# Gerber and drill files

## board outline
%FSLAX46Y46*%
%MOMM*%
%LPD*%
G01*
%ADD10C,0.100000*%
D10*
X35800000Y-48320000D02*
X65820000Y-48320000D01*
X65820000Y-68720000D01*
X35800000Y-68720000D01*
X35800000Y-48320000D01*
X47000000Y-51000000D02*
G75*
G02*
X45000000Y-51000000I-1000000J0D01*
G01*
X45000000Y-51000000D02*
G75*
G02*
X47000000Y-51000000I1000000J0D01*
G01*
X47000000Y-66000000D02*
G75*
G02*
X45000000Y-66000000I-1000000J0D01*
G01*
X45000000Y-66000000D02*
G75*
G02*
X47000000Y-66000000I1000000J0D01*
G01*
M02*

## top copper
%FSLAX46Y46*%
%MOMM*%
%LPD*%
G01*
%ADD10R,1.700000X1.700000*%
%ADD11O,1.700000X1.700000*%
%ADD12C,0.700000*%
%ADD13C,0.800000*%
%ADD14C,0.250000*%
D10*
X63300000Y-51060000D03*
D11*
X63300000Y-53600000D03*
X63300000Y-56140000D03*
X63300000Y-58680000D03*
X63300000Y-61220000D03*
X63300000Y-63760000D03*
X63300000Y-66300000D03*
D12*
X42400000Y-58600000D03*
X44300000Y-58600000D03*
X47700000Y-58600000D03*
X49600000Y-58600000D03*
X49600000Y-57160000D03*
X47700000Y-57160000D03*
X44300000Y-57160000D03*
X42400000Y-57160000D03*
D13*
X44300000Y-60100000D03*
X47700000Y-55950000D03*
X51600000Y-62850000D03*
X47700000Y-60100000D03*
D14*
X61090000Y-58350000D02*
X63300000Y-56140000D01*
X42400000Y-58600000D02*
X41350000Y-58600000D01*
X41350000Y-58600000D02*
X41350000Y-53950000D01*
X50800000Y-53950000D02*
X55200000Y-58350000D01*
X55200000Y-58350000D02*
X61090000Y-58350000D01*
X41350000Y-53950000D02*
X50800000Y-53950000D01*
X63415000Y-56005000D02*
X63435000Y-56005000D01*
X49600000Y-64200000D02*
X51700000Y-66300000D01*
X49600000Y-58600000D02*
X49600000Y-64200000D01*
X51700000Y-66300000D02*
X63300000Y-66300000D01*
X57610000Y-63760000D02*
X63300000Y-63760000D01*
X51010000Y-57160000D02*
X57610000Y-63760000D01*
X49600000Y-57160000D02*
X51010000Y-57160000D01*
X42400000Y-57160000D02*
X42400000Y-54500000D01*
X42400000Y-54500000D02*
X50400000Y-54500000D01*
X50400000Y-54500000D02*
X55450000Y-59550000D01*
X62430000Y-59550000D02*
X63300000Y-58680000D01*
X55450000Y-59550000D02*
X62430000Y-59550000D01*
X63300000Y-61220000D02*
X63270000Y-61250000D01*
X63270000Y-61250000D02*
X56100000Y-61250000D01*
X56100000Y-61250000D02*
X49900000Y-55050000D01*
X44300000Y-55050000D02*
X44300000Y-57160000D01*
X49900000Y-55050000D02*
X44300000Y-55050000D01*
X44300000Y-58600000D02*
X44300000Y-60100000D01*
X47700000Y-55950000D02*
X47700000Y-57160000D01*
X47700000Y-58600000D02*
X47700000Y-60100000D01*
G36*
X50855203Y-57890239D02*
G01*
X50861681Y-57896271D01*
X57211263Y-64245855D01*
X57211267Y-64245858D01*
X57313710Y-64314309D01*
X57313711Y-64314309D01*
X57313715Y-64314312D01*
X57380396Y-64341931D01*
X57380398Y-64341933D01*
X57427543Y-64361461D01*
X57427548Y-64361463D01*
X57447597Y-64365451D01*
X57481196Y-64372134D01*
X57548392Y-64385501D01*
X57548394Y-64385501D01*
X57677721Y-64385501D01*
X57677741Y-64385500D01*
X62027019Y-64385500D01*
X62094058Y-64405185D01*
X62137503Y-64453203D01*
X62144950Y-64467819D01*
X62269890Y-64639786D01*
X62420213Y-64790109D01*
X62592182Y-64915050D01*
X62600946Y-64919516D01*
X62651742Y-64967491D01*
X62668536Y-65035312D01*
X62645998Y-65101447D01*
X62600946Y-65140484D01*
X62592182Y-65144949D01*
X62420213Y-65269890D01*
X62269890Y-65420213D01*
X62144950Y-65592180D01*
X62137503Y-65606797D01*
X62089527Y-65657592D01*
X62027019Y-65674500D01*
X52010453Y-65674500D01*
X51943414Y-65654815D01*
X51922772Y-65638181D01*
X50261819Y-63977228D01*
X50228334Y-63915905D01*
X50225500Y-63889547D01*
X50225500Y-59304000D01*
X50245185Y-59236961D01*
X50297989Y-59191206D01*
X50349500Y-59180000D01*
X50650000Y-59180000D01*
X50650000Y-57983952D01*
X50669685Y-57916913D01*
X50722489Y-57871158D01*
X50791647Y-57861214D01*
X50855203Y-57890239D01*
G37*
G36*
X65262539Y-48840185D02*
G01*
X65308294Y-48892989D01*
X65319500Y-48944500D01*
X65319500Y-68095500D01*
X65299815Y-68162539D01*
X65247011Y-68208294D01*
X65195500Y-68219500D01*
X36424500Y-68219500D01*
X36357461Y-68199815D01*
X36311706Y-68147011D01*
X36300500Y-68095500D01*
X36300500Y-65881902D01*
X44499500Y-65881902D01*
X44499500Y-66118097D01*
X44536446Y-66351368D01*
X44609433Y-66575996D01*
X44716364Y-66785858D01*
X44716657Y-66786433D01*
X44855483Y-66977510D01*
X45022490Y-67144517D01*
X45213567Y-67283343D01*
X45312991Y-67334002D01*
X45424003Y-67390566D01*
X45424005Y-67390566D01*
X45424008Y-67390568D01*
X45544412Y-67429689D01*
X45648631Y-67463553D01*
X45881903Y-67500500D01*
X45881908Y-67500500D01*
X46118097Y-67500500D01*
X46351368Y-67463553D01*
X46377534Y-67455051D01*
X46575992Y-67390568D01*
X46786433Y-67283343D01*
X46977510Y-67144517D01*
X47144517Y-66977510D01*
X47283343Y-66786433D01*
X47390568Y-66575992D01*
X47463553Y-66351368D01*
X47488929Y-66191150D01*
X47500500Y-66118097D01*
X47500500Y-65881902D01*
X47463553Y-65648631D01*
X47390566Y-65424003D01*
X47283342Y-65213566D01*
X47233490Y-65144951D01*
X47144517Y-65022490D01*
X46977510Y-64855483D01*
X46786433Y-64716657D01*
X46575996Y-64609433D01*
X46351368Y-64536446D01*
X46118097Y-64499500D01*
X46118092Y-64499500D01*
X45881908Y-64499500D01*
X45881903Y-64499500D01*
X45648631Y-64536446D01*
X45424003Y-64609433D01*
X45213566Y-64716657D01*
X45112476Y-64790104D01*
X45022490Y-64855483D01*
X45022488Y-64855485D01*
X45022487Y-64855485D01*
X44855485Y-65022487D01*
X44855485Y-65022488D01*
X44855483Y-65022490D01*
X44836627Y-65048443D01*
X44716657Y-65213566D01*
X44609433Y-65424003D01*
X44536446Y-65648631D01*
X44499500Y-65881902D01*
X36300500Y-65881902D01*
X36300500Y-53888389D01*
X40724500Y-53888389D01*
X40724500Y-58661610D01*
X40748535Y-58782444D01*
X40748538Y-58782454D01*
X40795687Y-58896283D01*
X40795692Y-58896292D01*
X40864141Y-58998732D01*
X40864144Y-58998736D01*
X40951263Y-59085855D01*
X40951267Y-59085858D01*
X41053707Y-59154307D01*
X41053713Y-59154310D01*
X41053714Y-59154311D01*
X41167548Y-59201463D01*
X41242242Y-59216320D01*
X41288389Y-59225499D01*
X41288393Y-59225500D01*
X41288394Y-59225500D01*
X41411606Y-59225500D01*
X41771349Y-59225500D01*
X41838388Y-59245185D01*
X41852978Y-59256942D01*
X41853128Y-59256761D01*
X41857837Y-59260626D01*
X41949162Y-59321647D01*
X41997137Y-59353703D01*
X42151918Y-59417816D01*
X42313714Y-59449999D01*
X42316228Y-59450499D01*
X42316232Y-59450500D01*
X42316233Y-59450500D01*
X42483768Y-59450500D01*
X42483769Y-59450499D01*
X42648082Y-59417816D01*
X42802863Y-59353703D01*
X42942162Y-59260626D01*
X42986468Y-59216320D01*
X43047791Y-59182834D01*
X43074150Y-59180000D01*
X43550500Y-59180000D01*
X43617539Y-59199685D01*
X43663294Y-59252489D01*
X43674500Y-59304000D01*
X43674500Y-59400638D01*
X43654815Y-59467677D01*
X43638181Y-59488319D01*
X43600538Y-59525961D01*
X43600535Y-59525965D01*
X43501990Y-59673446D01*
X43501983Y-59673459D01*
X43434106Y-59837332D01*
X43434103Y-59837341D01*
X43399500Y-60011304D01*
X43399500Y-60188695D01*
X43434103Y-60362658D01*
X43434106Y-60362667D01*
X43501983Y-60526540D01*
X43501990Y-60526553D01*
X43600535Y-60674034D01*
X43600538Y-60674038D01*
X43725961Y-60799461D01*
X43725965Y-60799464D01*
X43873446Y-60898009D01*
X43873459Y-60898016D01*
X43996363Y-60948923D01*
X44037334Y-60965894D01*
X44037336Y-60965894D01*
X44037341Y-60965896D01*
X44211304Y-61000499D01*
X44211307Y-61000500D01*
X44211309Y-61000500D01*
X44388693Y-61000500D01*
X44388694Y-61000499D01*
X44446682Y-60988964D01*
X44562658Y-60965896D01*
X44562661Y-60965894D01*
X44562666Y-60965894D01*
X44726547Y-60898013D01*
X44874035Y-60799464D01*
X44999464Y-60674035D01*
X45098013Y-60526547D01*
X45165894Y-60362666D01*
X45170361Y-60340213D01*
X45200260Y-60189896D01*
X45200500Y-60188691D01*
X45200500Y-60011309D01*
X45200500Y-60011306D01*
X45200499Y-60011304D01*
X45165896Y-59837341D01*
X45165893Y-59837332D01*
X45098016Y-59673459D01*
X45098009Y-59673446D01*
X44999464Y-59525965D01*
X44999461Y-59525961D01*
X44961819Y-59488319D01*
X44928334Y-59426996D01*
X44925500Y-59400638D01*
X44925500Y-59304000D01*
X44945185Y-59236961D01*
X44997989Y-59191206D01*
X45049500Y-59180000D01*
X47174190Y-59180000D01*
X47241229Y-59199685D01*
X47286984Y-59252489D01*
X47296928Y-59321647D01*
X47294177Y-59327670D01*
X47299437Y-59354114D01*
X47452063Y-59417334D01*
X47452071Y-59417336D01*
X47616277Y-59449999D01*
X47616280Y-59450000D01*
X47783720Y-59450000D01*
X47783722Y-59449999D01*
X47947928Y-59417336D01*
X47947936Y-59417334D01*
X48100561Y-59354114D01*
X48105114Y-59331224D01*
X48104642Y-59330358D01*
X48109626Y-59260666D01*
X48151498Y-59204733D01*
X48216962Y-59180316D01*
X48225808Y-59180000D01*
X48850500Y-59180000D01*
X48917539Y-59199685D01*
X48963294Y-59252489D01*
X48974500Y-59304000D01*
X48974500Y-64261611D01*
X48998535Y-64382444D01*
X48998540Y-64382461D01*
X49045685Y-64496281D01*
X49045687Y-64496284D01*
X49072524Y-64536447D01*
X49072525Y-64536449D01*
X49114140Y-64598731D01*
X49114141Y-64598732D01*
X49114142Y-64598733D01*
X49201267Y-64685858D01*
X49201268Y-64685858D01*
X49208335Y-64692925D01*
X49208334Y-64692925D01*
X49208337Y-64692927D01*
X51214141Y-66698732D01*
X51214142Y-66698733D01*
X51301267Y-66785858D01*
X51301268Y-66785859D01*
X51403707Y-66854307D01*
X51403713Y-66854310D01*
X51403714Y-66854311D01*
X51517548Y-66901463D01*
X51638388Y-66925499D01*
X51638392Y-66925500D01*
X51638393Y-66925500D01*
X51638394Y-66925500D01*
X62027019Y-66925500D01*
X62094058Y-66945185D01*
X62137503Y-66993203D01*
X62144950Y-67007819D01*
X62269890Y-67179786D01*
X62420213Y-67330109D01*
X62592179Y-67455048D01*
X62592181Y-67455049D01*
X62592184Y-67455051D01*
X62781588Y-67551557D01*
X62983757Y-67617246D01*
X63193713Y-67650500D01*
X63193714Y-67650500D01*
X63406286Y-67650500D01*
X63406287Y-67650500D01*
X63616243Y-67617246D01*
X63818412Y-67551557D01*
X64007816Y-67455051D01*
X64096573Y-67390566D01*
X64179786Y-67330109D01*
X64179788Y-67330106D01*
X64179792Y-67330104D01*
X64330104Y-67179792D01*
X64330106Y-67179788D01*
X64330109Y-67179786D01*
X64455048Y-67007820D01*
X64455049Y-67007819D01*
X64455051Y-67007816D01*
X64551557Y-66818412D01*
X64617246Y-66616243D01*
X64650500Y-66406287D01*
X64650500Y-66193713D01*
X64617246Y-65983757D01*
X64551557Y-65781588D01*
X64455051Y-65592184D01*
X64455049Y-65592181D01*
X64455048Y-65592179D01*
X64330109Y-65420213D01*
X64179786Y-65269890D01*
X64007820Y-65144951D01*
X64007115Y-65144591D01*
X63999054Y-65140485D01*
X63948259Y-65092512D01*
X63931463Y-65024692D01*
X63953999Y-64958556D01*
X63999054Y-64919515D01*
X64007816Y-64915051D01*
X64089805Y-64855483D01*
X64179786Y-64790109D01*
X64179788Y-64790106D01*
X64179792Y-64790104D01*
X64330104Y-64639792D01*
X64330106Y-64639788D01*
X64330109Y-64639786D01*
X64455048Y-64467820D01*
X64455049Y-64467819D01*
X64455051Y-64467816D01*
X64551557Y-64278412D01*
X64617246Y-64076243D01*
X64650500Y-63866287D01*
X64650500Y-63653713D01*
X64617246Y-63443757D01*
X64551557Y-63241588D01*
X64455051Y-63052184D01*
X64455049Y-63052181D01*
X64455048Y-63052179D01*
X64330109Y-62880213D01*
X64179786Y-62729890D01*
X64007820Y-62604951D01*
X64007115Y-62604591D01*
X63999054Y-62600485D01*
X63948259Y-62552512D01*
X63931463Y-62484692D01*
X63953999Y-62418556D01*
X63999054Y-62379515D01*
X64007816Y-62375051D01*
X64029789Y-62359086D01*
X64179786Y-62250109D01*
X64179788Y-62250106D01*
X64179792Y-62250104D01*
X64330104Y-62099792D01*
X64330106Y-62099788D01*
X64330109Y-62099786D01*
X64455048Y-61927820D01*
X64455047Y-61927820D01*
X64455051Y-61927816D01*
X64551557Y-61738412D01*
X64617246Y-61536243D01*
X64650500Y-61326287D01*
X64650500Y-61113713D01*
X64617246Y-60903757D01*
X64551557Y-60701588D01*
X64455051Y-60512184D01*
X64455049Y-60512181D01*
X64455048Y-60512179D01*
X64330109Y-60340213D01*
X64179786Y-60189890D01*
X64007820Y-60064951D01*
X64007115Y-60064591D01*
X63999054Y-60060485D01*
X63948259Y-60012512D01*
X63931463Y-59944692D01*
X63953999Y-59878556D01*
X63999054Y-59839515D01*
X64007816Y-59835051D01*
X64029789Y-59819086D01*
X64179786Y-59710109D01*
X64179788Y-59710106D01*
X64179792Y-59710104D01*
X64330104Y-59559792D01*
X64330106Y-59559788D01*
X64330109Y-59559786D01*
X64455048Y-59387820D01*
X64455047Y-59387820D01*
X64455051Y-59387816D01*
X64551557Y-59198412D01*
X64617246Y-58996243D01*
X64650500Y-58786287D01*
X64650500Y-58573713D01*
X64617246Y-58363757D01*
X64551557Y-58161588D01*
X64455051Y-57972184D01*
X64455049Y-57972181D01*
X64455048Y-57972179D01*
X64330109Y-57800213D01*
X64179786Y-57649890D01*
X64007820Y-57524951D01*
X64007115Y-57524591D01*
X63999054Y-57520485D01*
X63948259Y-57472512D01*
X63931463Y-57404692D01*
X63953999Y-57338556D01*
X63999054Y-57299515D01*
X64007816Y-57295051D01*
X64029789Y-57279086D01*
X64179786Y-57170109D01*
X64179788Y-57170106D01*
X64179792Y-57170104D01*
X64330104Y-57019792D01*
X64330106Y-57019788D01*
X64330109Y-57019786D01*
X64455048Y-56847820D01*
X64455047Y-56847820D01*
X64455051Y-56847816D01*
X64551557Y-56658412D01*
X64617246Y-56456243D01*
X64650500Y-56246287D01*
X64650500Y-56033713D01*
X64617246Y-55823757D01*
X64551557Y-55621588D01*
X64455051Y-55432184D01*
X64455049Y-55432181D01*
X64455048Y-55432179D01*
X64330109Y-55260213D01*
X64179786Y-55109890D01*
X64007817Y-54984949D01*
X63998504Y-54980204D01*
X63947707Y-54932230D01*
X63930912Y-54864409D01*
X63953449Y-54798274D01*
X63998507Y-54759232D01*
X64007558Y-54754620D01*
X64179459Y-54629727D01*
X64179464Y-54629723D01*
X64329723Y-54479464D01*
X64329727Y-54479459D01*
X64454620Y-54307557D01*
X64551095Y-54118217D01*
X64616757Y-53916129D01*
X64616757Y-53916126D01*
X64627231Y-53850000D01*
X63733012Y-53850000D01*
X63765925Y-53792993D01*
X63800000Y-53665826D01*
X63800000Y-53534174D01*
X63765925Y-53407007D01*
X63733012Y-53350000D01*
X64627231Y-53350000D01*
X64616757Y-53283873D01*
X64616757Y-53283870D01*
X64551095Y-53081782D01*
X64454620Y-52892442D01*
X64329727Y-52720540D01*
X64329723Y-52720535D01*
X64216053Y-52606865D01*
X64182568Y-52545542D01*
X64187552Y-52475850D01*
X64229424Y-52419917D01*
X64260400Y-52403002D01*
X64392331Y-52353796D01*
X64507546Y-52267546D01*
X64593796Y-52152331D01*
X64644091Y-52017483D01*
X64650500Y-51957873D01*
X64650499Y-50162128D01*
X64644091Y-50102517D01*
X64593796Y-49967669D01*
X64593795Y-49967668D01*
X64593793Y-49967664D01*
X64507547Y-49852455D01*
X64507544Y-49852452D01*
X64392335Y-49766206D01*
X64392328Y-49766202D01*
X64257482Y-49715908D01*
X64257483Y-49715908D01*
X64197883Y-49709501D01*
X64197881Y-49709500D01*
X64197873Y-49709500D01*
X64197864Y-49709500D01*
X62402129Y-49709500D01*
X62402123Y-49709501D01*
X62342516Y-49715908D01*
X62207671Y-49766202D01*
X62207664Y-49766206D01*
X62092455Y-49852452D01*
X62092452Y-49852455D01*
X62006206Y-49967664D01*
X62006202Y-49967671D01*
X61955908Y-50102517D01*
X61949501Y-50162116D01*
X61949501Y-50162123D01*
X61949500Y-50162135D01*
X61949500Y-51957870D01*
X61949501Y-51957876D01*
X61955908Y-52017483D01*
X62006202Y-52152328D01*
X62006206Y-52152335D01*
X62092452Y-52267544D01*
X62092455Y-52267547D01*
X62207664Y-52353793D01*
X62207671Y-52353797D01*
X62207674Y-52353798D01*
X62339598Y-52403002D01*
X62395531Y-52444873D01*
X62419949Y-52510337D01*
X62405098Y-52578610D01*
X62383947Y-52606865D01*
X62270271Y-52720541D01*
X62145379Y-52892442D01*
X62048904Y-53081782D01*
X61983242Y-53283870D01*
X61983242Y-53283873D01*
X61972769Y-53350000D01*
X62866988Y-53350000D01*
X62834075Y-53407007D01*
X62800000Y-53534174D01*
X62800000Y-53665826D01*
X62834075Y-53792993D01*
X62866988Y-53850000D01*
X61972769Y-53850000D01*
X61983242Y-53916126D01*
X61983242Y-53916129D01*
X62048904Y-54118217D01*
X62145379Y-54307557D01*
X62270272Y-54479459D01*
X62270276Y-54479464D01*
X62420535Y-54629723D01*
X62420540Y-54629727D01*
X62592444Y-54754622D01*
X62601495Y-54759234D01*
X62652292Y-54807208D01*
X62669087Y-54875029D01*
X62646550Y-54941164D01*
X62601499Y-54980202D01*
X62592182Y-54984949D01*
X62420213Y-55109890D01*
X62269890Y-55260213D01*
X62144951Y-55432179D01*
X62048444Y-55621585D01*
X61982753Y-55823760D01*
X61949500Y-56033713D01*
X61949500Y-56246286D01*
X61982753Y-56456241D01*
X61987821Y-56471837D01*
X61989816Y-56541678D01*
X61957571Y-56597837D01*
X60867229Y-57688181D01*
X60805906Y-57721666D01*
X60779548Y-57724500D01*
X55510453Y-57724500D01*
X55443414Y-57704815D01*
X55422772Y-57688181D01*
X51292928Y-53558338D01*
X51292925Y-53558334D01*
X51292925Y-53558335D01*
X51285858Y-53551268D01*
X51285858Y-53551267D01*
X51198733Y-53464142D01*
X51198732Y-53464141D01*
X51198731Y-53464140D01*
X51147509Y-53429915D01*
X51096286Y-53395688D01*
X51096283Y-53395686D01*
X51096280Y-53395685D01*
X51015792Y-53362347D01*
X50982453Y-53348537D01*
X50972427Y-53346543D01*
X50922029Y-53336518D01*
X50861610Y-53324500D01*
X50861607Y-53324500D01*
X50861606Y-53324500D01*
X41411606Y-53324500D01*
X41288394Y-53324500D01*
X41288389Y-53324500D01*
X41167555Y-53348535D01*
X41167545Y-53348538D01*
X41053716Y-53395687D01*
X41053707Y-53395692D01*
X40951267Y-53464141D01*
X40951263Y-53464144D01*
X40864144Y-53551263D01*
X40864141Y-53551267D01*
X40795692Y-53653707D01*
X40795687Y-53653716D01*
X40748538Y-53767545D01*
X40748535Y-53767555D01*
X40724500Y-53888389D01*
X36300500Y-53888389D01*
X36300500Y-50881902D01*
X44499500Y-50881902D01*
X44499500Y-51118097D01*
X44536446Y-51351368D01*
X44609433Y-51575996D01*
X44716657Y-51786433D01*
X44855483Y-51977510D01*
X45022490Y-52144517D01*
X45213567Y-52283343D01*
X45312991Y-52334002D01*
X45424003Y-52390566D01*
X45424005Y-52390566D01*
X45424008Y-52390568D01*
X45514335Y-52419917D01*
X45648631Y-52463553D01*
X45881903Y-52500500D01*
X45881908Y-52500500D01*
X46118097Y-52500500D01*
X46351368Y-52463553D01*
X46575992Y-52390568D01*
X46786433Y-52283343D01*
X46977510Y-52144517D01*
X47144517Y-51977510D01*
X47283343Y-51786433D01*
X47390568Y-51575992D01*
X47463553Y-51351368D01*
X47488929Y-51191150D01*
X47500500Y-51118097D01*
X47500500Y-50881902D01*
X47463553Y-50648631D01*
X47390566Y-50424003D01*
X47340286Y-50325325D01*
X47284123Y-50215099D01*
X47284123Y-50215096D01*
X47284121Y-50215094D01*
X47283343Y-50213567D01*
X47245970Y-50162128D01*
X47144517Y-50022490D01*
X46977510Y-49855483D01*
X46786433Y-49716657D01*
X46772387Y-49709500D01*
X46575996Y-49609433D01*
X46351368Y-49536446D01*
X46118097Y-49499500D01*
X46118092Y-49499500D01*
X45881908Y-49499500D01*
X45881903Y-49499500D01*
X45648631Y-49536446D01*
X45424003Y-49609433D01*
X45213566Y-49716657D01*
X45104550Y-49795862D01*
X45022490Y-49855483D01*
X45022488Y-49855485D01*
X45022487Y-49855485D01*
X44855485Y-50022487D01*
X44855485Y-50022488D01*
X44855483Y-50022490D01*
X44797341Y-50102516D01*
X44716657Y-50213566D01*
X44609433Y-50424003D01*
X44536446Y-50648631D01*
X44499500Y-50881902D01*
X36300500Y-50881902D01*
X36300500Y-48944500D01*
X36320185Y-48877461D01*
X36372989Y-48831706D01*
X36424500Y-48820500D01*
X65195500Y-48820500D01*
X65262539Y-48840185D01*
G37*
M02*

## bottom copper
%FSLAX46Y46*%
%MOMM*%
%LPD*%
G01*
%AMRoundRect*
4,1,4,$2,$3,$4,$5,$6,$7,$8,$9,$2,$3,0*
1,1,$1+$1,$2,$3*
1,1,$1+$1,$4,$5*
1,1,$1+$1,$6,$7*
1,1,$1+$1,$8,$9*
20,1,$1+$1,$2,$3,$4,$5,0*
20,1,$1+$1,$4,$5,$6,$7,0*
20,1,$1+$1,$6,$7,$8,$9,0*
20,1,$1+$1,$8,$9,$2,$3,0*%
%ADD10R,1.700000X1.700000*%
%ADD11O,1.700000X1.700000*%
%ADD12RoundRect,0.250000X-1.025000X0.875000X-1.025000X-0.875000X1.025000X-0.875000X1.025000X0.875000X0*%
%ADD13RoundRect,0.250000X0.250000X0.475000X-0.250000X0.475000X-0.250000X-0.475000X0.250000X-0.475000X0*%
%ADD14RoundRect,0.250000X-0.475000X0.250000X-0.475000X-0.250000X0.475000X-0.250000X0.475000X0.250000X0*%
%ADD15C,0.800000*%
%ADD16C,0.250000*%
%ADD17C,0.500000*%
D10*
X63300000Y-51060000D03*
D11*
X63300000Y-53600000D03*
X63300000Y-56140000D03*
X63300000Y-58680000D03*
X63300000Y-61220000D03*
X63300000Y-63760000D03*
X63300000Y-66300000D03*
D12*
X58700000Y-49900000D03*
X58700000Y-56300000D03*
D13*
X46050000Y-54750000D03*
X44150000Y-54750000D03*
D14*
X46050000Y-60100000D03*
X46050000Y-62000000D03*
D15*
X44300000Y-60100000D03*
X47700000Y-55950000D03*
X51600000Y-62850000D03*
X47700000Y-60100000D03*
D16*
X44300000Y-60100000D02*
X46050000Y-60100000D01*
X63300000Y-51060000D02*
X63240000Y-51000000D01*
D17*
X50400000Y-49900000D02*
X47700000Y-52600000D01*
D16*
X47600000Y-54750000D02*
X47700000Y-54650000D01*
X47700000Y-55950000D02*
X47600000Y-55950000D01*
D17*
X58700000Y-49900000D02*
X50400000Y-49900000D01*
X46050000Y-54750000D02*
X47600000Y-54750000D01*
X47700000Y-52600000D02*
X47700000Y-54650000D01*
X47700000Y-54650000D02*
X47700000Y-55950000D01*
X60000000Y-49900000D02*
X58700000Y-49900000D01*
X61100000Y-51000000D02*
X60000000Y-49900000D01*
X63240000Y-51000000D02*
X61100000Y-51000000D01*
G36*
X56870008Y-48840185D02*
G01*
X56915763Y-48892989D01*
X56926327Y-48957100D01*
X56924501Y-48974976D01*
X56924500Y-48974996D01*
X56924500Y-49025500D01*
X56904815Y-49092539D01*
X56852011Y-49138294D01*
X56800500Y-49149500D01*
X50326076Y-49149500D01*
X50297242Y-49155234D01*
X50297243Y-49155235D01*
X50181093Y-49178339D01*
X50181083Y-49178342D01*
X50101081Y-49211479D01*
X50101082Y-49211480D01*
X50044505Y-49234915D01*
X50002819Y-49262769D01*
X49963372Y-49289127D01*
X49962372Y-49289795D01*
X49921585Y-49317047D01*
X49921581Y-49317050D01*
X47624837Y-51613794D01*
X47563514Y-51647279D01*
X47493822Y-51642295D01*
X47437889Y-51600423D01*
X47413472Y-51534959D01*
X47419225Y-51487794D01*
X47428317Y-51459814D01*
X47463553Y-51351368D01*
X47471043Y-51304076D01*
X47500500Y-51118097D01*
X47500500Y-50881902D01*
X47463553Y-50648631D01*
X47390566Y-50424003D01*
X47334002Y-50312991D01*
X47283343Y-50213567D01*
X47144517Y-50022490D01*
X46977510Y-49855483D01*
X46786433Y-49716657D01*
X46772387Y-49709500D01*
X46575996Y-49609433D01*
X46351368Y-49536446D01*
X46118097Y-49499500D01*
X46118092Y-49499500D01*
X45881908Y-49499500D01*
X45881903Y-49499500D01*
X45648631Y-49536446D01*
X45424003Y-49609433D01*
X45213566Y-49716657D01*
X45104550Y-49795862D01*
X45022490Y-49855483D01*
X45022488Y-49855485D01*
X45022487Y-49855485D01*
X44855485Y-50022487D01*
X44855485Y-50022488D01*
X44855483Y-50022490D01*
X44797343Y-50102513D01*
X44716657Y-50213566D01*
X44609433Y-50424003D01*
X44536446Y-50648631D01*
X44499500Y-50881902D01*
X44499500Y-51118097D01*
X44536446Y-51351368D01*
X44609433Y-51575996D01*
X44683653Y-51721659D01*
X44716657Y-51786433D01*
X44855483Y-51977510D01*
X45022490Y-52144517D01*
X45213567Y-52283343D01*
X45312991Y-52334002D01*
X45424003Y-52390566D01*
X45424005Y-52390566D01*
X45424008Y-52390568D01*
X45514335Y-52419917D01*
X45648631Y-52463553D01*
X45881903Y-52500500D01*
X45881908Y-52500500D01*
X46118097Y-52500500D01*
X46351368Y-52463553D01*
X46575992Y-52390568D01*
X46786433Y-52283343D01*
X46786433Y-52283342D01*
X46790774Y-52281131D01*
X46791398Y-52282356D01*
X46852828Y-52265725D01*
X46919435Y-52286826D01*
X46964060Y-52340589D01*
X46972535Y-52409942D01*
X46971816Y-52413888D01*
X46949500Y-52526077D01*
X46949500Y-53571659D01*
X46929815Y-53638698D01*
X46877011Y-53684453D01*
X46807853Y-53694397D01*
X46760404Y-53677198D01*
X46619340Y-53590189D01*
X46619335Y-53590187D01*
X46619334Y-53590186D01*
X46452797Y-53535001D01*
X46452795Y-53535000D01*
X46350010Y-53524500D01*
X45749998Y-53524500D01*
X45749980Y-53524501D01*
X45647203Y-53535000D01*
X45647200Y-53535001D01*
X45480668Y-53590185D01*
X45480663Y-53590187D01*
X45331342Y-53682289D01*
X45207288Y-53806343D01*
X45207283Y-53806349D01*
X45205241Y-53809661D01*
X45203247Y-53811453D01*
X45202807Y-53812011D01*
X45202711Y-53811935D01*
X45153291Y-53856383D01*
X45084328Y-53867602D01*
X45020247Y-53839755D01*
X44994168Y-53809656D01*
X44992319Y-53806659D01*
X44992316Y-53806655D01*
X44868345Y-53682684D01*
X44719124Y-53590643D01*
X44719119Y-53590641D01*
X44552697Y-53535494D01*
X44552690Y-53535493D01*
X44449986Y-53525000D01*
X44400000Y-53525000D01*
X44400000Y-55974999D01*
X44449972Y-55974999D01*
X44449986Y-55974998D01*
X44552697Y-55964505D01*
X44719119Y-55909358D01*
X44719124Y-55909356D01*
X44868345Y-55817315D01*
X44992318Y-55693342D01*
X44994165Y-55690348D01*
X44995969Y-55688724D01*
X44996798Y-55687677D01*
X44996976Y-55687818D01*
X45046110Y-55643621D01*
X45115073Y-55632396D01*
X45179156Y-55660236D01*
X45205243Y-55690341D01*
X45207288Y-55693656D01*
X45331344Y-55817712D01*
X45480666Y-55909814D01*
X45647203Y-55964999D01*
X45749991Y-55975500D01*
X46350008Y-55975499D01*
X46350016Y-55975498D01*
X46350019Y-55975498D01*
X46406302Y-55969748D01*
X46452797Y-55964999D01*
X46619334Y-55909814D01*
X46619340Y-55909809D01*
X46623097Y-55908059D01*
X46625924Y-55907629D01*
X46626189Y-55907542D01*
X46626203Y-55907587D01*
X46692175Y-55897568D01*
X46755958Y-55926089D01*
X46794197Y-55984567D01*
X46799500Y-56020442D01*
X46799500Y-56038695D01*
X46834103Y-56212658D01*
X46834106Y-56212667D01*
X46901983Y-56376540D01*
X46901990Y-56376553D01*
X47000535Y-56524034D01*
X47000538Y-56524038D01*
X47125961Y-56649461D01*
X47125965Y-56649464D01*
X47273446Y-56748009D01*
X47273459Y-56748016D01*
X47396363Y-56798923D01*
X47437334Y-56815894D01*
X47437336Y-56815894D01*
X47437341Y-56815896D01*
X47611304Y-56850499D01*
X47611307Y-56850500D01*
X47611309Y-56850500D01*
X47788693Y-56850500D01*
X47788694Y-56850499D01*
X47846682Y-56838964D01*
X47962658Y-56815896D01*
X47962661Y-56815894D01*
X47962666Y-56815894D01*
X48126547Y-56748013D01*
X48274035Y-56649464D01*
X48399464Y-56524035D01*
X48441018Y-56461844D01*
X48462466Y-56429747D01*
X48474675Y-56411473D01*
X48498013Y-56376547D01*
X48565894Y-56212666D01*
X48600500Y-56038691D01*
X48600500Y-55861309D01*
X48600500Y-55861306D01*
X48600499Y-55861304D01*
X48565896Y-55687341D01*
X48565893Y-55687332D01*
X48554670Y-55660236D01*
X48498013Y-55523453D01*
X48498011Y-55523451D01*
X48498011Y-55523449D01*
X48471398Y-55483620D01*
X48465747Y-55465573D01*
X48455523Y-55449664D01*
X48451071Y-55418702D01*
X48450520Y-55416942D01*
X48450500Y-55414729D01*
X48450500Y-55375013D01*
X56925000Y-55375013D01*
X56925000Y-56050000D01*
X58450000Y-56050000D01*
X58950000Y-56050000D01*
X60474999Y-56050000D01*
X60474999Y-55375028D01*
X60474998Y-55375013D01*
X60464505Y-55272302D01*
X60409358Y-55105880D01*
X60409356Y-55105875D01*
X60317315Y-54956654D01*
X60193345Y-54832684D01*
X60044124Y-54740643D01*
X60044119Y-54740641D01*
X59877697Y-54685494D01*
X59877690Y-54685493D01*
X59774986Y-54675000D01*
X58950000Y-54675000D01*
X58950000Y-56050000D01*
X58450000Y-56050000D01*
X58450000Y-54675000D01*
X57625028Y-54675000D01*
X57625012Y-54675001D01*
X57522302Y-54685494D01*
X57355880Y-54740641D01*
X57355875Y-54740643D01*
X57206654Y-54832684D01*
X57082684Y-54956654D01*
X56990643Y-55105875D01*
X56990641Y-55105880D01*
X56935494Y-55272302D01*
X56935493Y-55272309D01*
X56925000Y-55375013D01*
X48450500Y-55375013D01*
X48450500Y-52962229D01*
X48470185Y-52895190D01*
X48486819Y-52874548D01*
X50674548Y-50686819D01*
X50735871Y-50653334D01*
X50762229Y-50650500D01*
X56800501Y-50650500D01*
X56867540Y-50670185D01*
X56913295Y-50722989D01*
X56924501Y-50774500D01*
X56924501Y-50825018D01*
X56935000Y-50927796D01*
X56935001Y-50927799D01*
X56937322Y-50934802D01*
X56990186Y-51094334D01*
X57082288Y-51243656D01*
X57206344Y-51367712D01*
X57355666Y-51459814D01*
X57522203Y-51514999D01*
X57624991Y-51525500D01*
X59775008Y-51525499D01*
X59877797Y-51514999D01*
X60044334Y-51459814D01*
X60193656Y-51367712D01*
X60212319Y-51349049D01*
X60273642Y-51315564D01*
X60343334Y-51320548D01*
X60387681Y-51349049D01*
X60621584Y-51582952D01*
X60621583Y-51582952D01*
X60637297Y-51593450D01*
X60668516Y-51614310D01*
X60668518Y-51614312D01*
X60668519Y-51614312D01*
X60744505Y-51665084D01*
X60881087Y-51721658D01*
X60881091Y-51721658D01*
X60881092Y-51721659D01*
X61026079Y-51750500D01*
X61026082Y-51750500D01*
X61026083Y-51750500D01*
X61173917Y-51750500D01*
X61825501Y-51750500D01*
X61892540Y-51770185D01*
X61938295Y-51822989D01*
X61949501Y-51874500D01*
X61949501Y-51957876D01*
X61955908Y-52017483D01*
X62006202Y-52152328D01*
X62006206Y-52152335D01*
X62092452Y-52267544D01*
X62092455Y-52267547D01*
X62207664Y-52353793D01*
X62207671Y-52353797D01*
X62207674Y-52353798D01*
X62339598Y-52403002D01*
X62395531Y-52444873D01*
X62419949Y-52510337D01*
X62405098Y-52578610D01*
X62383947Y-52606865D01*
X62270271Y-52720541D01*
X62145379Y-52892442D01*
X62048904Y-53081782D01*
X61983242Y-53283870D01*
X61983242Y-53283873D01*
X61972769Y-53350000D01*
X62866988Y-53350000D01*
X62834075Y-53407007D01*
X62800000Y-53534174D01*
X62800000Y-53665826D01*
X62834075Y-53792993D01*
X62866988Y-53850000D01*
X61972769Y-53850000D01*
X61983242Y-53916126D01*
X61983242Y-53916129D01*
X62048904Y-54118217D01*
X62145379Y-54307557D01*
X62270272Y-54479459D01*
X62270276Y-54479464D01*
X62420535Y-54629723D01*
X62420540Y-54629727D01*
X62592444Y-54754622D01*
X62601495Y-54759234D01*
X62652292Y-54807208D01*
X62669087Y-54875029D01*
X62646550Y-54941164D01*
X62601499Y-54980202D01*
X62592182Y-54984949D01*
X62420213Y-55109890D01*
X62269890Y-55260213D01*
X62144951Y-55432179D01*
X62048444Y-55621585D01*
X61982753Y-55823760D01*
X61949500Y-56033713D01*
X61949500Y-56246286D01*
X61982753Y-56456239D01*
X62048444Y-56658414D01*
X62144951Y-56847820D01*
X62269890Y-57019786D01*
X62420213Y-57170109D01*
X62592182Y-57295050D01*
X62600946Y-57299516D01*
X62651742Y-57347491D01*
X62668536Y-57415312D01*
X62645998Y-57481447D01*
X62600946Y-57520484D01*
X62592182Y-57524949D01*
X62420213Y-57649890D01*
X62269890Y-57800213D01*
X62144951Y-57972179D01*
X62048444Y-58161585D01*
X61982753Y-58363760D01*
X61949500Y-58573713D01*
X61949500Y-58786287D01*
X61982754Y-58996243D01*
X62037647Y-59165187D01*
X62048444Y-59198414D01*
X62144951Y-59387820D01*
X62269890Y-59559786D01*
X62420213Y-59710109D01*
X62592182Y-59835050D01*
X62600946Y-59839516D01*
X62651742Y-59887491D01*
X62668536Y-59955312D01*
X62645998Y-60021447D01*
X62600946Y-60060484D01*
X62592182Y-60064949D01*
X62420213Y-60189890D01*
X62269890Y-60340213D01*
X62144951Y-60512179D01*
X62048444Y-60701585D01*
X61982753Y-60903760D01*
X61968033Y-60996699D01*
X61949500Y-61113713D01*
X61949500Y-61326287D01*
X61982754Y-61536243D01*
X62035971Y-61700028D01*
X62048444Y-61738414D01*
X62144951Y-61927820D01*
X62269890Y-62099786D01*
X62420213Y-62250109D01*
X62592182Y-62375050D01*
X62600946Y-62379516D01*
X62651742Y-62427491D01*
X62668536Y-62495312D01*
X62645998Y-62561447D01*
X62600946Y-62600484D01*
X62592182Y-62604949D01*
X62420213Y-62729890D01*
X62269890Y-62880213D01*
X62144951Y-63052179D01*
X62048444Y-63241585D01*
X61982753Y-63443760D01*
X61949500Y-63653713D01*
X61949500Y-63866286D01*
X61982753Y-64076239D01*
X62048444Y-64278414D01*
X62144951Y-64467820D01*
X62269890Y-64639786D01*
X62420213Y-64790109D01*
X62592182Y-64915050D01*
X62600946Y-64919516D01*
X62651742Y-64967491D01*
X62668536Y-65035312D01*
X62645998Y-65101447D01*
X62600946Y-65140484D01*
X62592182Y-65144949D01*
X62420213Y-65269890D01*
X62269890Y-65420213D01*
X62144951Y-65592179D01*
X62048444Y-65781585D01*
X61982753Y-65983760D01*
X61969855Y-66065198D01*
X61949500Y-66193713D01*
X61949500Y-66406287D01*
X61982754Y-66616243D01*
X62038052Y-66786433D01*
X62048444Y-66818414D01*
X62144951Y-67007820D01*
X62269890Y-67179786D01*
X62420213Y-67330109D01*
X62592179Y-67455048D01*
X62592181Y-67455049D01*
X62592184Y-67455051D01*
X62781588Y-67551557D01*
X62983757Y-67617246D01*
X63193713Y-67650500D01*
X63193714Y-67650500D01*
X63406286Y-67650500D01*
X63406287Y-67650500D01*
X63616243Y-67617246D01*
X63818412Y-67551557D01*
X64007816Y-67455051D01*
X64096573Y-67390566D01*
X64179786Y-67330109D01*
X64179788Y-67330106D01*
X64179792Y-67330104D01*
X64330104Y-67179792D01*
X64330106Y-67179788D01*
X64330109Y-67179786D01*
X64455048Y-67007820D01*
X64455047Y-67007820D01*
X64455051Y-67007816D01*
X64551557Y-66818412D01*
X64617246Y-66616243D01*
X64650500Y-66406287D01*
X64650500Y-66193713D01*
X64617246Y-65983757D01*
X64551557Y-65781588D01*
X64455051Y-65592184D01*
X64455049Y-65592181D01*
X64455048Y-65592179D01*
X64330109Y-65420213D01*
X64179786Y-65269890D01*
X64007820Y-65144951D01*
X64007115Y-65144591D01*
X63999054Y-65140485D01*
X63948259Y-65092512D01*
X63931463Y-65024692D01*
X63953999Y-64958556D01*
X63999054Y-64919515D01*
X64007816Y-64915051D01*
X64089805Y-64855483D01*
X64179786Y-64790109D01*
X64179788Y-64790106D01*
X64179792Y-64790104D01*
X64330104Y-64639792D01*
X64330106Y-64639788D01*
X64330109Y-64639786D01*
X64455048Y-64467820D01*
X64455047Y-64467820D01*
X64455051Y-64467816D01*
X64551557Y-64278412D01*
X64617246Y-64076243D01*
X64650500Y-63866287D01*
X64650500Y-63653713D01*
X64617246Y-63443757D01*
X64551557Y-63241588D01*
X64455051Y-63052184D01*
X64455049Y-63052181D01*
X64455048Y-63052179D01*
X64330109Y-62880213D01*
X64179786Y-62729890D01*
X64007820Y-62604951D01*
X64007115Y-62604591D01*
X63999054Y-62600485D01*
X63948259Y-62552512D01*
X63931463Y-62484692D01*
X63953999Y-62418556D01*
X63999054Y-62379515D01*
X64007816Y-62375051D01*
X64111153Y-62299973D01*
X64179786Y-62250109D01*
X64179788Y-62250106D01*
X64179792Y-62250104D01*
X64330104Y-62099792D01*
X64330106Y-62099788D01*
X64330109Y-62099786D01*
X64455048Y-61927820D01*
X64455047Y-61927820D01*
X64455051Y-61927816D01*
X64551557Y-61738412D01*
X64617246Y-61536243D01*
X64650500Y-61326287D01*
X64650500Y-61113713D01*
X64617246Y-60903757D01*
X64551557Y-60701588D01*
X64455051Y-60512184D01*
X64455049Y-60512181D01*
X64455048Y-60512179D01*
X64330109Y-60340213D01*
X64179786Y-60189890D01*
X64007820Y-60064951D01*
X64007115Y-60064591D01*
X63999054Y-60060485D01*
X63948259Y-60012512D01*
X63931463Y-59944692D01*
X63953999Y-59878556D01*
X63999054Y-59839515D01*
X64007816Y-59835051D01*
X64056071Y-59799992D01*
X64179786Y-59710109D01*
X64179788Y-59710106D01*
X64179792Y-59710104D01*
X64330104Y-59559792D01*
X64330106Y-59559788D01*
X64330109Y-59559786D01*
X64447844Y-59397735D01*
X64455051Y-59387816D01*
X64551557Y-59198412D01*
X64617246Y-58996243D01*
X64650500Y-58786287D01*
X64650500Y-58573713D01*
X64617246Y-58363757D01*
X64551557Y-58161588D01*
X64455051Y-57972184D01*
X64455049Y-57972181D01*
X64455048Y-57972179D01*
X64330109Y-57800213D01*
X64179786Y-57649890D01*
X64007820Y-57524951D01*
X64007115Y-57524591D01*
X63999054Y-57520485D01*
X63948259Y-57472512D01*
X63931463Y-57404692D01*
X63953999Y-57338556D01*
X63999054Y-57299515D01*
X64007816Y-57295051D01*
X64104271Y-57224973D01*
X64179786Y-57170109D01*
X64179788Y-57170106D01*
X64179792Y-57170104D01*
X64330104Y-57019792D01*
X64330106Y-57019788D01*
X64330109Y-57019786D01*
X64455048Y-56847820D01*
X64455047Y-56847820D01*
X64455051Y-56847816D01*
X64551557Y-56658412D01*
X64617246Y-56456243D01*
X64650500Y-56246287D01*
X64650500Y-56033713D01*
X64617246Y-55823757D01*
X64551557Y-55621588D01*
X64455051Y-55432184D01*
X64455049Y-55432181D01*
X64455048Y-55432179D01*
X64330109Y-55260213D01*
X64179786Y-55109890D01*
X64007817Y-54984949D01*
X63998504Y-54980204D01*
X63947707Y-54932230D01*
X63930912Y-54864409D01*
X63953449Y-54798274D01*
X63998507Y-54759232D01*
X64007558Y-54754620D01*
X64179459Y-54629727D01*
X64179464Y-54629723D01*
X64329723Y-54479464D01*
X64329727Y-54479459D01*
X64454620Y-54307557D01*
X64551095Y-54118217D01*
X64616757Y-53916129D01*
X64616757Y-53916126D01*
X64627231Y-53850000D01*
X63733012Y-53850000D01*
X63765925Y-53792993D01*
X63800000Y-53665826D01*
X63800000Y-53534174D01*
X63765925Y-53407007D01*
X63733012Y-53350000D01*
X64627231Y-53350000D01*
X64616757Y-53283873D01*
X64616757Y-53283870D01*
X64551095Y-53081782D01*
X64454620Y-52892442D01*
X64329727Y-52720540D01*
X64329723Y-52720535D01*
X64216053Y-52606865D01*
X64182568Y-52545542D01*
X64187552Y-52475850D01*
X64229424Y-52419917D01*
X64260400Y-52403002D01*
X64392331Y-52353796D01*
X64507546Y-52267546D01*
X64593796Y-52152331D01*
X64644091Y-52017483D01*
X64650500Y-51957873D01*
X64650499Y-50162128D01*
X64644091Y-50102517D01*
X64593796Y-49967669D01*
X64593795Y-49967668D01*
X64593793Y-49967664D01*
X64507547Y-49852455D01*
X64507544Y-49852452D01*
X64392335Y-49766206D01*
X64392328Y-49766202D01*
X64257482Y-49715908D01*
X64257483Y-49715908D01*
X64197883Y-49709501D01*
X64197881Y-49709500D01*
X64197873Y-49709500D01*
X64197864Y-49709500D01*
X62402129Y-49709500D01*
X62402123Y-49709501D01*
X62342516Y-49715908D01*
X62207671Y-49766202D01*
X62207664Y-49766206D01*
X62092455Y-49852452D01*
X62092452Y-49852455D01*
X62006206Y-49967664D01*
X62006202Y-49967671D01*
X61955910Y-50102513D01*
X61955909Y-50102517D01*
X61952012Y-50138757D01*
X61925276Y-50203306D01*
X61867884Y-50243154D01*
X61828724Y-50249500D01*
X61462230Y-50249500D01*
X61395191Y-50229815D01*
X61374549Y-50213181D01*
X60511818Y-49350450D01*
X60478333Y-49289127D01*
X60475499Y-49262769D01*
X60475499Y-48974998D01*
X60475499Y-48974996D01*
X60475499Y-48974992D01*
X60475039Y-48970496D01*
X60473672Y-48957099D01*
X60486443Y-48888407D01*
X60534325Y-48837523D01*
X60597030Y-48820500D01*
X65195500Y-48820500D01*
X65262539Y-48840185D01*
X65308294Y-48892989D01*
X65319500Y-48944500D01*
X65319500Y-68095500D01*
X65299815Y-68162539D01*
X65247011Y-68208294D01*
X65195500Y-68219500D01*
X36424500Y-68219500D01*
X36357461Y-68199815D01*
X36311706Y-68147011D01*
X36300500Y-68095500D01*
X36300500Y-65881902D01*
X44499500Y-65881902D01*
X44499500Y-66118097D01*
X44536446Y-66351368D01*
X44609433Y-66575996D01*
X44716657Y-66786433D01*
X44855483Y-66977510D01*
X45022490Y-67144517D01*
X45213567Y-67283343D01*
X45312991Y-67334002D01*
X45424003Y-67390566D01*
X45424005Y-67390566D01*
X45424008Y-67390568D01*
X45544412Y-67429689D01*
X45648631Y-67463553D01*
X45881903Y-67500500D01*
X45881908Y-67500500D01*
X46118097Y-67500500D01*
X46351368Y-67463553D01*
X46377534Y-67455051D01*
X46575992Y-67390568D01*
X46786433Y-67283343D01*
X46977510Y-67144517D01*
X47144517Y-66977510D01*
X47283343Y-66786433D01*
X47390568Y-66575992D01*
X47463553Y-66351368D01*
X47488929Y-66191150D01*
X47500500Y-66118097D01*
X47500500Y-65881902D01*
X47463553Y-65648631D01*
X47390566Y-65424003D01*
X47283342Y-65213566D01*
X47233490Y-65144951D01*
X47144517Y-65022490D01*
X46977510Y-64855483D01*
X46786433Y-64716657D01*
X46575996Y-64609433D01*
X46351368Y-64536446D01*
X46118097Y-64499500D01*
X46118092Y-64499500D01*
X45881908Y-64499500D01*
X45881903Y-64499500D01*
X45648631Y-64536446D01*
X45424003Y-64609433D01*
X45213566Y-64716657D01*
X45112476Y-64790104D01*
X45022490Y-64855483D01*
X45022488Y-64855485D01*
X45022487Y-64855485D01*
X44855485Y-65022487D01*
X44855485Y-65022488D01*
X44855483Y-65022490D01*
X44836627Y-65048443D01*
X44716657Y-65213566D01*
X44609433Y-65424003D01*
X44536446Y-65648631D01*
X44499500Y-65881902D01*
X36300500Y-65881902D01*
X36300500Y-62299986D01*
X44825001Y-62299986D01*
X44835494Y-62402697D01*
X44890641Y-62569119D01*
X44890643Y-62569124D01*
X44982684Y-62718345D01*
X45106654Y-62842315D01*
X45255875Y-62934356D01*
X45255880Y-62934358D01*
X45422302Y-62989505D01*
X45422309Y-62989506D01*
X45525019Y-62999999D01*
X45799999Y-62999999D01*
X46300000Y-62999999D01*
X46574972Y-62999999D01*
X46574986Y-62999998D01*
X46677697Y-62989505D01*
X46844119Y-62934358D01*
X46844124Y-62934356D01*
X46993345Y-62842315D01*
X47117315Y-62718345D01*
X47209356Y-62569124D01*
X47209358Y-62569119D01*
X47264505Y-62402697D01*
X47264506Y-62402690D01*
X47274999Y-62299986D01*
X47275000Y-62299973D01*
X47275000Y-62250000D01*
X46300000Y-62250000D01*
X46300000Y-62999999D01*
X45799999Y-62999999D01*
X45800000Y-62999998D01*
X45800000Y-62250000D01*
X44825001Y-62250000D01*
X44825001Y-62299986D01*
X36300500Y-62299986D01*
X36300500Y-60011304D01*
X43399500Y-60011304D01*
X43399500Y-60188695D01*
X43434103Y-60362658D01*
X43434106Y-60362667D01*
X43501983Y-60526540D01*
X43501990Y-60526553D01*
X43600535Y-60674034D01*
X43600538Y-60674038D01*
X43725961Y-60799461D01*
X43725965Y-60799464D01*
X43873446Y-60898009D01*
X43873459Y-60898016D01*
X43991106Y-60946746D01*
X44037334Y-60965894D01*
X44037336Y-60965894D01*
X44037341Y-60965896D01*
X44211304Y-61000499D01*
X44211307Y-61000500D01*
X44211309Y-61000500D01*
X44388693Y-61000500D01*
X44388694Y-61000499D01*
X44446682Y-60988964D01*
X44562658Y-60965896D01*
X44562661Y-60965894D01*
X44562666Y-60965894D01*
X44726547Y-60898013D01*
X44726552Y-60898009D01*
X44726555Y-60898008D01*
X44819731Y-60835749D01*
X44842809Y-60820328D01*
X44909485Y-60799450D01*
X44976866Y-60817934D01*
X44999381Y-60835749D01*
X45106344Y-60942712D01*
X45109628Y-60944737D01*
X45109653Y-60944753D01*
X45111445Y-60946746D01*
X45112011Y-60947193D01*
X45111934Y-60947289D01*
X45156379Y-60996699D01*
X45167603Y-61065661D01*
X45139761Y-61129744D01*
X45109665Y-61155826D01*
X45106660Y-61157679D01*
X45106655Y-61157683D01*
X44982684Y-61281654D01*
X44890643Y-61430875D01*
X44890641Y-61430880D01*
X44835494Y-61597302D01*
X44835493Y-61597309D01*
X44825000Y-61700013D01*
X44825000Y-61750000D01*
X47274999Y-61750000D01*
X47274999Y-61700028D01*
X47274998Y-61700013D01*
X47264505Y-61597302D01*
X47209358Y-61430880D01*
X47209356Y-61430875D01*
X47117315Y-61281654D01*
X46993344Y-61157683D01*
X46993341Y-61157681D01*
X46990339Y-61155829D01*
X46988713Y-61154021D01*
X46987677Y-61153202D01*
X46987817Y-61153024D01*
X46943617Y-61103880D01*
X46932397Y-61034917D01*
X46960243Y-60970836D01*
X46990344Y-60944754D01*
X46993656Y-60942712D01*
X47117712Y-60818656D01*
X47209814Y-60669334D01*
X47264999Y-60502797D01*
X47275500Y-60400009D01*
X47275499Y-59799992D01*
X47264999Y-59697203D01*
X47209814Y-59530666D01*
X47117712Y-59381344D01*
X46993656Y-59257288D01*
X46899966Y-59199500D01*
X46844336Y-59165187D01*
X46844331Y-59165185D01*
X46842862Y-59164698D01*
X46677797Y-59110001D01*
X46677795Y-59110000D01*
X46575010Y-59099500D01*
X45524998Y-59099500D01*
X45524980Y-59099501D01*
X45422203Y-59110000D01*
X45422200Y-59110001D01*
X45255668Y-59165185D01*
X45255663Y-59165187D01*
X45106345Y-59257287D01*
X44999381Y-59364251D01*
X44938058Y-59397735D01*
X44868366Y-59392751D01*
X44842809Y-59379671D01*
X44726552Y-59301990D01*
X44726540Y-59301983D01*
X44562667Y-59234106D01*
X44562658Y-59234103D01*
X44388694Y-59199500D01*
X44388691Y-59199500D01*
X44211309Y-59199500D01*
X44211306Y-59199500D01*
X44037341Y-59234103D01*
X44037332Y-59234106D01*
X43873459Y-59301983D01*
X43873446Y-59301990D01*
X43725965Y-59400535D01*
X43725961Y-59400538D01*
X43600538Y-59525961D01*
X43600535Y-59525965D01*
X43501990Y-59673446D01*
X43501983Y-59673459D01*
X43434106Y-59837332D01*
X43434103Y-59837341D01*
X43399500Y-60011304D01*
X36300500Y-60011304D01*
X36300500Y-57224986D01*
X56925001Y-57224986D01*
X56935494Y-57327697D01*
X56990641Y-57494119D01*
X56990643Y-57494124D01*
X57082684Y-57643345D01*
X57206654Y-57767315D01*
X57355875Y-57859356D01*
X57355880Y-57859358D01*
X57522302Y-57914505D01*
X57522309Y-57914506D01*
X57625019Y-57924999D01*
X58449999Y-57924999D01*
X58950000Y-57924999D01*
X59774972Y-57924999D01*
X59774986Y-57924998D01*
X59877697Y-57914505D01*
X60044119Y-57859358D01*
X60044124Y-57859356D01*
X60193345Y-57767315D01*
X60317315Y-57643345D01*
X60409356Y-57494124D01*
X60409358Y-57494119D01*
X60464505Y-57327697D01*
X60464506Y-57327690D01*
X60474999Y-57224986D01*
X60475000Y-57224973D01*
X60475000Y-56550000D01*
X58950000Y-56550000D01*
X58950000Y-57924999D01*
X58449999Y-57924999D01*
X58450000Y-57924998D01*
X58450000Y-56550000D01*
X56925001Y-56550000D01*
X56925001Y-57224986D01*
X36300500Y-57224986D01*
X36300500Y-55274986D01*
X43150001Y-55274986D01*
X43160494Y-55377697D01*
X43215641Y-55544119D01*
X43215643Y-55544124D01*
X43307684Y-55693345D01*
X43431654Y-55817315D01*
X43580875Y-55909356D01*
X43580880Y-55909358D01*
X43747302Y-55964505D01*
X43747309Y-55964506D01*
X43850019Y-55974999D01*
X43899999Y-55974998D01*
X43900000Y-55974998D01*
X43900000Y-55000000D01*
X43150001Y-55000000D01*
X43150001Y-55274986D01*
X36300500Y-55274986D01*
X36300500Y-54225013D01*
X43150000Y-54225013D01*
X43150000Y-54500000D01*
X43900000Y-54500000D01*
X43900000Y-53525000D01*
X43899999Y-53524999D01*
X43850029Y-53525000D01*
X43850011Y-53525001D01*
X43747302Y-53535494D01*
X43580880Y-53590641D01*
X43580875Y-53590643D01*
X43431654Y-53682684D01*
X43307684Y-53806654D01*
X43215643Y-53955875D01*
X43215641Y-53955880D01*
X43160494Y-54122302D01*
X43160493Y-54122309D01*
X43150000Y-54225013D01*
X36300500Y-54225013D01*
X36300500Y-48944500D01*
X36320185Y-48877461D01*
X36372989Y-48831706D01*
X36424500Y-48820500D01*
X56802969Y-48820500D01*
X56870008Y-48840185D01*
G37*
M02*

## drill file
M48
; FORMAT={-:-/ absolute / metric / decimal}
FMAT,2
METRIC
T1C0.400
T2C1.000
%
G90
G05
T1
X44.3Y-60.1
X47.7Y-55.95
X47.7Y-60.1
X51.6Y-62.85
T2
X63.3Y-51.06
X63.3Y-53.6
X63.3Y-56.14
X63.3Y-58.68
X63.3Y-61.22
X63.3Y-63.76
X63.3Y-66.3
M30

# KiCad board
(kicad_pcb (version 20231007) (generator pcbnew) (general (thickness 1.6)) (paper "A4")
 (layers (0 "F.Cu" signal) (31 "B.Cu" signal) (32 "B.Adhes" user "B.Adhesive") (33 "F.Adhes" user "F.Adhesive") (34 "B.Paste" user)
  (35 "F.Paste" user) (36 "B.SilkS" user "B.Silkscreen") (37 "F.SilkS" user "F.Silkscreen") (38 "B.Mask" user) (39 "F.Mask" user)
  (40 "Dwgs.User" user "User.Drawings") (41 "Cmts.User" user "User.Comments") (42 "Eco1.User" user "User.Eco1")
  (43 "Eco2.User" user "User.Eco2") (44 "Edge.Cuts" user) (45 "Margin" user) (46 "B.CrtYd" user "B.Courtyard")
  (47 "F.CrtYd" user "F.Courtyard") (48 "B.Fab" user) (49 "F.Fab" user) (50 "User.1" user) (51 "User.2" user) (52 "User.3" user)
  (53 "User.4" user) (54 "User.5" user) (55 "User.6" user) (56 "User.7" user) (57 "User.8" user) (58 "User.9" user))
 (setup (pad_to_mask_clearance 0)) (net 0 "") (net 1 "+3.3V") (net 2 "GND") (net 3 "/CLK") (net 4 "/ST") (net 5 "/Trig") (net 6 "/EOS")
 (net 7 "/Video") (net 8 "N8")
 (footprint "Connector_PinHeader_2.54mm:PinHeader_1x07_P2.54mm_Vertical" (layer "F.Cu") (at 63.3 51.06)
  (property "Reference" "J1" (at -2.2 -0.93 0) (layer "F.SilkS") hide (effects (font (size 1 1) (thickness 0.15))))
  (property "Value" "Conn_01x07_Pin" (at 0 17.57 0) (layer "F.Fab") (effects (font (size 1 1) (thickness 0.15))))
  (pad "1" thru_hole rect (at 0 0) (size 1.7 1.7) (drill 1) (layers "*.Cu" "*.Mask") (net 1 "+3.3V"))
  (pad "2" thru_hole oval (at 0 2.54) (size 1.7 1.7) (drill 1) (layers "*.Cu" "*.Mask") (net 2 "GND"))
  (pad "3" thru_hole oval (at 0 5.08) (size 1.7 1.7) (drill 1) (layers "*.Cu" "*.Mask") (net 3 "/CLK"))
  (pad "4" thru_hole oval (at 0 7.62) (size 1.7 1.7) (drill 1) (layers "*.Cu" "*.Mask") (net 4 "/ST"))
  (pad "5" thru_hole oval (at 0 10.16) (size 1.7 1.7) (drill 1) (layers "*.Cu" "*.Mask") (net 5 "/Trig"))
  (pad "6" thru_hole oval (at 0 12.7) (size 1.7 1.7) (drill 1) (layers "*.Cu" "*.Mask") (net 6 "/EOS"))
  (pad "7" thru_hole oval (at 0 15.24) (size 1.7 1.7) (drill 1) (layers "*.Cu" "*.Mask") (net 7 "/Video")))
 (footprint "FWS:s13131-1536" (layer "F.Cu") (at 46 57.88)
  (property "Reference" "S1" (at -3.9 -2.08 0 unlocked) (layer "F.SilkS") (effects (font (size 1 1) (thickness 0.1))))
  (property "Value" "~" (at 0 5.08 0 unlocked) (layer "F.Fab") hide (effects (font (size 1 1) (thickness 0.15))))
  (pad "1" smd circle (at -3.6 0.72) (size 0.7 0.7) (layers "F.Cu" "F.Paste" "F.Mask") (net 3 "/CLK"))
  (pad "2" smd circle (at -1.7 0.72) (size 0.7 0.7) (layers "F.Cu" "F.Paste" "F.Mask") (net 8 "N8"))
  (pad "3" smd circle (at 1.7 0.72) (size 0.7 0.7) (layers "F.Cu" "F.Paste" "F.Mask") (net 2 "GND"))
  (pad "4" smd circle (at 3.6 0.72) (size 0.7 0.7) (layers "F.Cu" "F.Paste" "F.Mask") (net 7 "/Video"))
  (pad "5" smd circle (at 3.6 -0.72) (size 0.7 0.7) (layers "F.Cu" "F.Paste" "F.Mask") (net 6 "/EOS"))
  (pad "6" smd circle (at 1.7 -0.72) (size 0.7 0.7) (layers "F.Cu" "F.Paste" "F.Mask") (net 1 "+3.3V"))
  (pad "7" smd circle (at -1.7 -0.72) (size 0.7 0.7) (layers "F.Cu" "F.Paste" "F.Mask") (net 5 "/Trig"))
  (pad "8" smd circle (at -3.6 -0.72) (size 0.7 0.7) (layers "F.Cu" "F.Paste" "F.Mask") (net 4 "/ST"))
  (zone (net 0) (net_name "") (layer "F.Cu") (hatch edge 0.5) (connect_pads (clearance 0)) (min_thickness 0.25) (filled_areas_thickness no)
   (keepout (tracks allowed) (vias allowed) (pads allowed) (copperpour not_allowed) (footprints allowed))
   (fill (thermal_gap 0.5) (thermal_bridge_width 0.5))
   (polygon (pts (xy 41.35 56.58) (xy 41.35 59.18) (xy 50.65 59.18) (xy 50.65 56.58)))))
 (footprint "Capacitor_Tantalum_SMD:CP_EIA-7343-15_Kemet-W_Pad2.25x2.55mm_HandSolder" (layer "B.Cu") (at 58.7 53.1 -90)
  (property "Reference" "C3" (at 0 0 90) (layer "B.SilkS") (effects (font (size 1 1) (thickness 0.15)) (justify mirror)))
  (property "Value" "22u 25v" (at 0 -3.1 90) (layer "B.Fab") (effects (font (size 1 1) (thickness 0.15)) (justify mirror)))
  (pad "1" smd roundrect (at -3.2 0 270) (size 2.25 2.55) (layers "B.Cu" "B.Paste" "B.Mask") (roundrect_rratio 0.1111111111) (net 1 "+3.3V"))
  (pad "2" smd roundrect (at 3.2 0 270) (size 2.25 2.55) (layers "B.Cu" "B.Paste" "B.Mask") (roundrect_rratio 0.1111111111) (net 2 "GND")))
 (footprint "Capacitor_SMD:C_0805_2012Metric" (layer "B.Cu") (at 45.1 54.75 180)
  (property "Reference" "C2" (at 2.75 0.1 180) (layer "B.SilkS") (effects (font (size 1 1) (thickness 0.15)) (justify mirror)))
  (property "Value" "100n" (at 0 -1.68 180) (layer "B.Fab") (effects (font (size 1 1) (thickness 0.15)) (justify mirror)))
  (pad "1" smd roundrect (at -0.95 0 180) (size 1 1.45) (layers "B.Cu" "B.Paste" "B.Mask") (roundrect_rratio 0.25) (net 1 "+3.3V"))
  (pad "2" smd roundrect (at 0.95 0 180) (size 1 1.45) (layers "B.Cu" "B.Paste" "B.Mask") (roundrect_rratio 0.25) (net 2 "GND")))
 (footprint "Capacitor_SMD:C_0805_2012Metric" (layer "B.Cu") (at 46.05 61.05 -90)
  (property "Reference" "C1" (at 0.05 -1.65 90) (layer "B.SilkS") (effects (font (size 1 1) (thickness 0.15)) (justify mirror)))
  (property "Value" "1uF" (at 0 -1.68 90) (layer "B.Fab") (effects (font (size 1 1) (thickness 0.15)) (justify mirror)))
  (pad "1" smd roundrect (at -0.95 0 270) (size 1 1.45) (layers "B.Cu" "B.Paste" "B.Mask") (roundrect_rratio 0.25) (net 8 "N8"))
  (pad "2" smd roundrect (at 0.95 0 270) (size 1 1.45) (layers "B.Cu" "B.Paste" "B.Mask") (roundrect_rratio 0.25) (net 2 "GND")))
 (gr_rect (start 35.8 48.32) (end 65.82 68.72) (stroke (width 0.1) (type default)) (fill none) (layer "Edge.Cuts"))
 (gr_circle (center 46 51) (end 47 51) (stroke (width 0.1) (type default)) (fill none) (layer "Edge.Cuts"))
 (gr_circle (center 46 66) (end 47 66) (stroke (width 0.1) (type default)) (fill none) (layer "Edge.Cuts"))
 (segment (start 61.09 58.35) (end 63.3 56.14) (width 0.25) (layer "F.Cu") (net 3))
 (segment (start 42.4 58.6) (end 41.35 58.6) (width 0.25) (layer "F.Cu") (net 3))
 (segment (start 41.35 58.6) (end 41.35 53.95) (width 0.25) (layer "F.Cu") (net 3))
 (segment (start 50.8 53.95) (end 55.2 58.35) (width 0.25) (layer "F.Cu") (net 3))
 (segment (start 55.2 58.35) (end 61.09 58.35) (width 0.25) (layer "F.Cu") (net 3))
 (segment (start 41.35 53.95) (end 50.8 53.95) (width 0.25) (layer "F.Cu") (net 3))
 (segment (start 63.415 56.005) (end 63.435 56.005) (width 0.25) (layer "F.Cu") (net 3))
 (segment (start 49.6 64.2) (end 51.7 66.3) (width 0.25) (layer "F.Cu") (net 7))
 (segment (start 49.6 58.6) (end 49.6 64.2) (width 0.25) (layer "F.Cu") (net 7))
 (segment (start 51.7 66.3) (end 63.3 66.3) (width 0.25) (layer "F.Cu") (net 7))
 (segment (start 57.61 63.76) (end 63.3 63.76) (width 0.25) (layer "F.Cu") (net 6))
 (segment (start 51.01 57.16) (end 57.61 63.76) (width 0.25) (layer "F.Cu") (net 6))
 (segment (start 49.6 57.16) (end 51.01 57.16) (width 0.25) (layer "F.Cu") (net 6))
 (segment (start 42.4 57.16) (end 42.4 54.5) (width 0.25) (layer "F.Cu") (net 4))
 (segment (start 42.4 54.5) (end 50.4 54.5) (width 0.25) (layer "F.Cu") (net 4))
 (segment (start 50.4 54.5) (end 55.45 59.55) (width 0.25) (layer "F.Cu") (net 4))
 (segment (start 62.43 59.55) (end 63.3 58.68) (width 0.25) (layer "F.Cu") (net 4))
 (segment (start 55.45 59.55) (end 62.43 59.55) (width 0.25) (layer "F.Cu") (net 4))
 (segment (start 63.3 61.22) (end 63.27 61.25) (width 0.25) (layer "F.Cu") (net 5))
 (segment (start 63.27 61.25) (end 56.1 61.25) (width 0.25) (layer "F.Cu") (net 5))
 (segment (start 56.1 61.25) (end 49.9 55.05) (width 0.25) (layer "F.Cu") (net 5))
 (segment (start 44.3 55.05) (end 44.3 57.16) (width 0.25) (layer "F.Cu") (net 5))
 (segment (start 49.9 55.05) (end 44.3 55.05) (width 0.25) (layer "F.Cu") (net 5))
 (segment (start 44.3 58.6) (end 44.3 60.1) (width 0.25) (layer "F.Cu") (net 8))
 (via (at 44.3 60.1) (size 0.8) (drill 0.4) (layers "F.Cu" "B.Cu") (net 8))
 (segment (start 44.3 60.1) (end 46.05 60.1) (width 0.25) (layer "B.Cu") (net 8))
 (segment (start 47.7 55.95) (end 47.7 57.16) (width 0.25) (layer "F.Cu") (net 1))
 (via (at 47.7 55.95) (size 0.8) (drill 0.4) (layers "F.Cu" "B.Cu") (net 1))
 (segment (start 63.3 51.06) (end 63.24 51) (width 0.25) (layer "B.Cu") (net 1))
 (segment (start 50.4 49.9) (end 47.7 52.6) (width 0.5) (layer "B.Cu") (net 1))
 (segment (start 47.6 54.75) (end 47.7 54.65) (width 0.25) (layer "B.Cu") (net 1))
 (segment (start 47.7 55.95) (end 47.6 55.95) (width 0.25) (layer "B.Cu") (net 1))
 (segment (start 58.7 49.9) (end 50.4 49.9) (width 0.5) (layer "B.Cu") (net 1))
 (segment (start 46.05 54.75) (end 47.6 54.75) (width 0.5) (layer "B.Cu") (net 1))
 (segment (start 47.7 52.6) (end 47.7 54.65) (width 0.5) (layer "B.Cu") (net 1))
 (segment (start 47.7 54.65) (end 47.7 55.95) (width 0.5) (layer "B.Cu") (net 1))
 (segment (start 60 49.9) (end 58.7 49.9) (width 0.5) (layer "B.Cu") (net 1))
 (segment (start 61.1 51) (end 60 49.9) (width 0.5) (layer "B.Cu") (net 1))
 (segment (start 63.24 51) (end 61.1 51) (width 0.5) (layer "B.Cu") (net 1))
 (segment (start 47.7 58.6) (end 47.7 60.1) (width 0.25) (layer "F.Cu") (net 2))
 (via (at 51.6 62.85) (size 0.8) (drill 0.4) (layers "F.Cu" "B.Cu") (free) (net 2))
 (via (at 47.7 60.1) (size 0.8) (drill 0.4) (layers "F.Cu" "B.Cu") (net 2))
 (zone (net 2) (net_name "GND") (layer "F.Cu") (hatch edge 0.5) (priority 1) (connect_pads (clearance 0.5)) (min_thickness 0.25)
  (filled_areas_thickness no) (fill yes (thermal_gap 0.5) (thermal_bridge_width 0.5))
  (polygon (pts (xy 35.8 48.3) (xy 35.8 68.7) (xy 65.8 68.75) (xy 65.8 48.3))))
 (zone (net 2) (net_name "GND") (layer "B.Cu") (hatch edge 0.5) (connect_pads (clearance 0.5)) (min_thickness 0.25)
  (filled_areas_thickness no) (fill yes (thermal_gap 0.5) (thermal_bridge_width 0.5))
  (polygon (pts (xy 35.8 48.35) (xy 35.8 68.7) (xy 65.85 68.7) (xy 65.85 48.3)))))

